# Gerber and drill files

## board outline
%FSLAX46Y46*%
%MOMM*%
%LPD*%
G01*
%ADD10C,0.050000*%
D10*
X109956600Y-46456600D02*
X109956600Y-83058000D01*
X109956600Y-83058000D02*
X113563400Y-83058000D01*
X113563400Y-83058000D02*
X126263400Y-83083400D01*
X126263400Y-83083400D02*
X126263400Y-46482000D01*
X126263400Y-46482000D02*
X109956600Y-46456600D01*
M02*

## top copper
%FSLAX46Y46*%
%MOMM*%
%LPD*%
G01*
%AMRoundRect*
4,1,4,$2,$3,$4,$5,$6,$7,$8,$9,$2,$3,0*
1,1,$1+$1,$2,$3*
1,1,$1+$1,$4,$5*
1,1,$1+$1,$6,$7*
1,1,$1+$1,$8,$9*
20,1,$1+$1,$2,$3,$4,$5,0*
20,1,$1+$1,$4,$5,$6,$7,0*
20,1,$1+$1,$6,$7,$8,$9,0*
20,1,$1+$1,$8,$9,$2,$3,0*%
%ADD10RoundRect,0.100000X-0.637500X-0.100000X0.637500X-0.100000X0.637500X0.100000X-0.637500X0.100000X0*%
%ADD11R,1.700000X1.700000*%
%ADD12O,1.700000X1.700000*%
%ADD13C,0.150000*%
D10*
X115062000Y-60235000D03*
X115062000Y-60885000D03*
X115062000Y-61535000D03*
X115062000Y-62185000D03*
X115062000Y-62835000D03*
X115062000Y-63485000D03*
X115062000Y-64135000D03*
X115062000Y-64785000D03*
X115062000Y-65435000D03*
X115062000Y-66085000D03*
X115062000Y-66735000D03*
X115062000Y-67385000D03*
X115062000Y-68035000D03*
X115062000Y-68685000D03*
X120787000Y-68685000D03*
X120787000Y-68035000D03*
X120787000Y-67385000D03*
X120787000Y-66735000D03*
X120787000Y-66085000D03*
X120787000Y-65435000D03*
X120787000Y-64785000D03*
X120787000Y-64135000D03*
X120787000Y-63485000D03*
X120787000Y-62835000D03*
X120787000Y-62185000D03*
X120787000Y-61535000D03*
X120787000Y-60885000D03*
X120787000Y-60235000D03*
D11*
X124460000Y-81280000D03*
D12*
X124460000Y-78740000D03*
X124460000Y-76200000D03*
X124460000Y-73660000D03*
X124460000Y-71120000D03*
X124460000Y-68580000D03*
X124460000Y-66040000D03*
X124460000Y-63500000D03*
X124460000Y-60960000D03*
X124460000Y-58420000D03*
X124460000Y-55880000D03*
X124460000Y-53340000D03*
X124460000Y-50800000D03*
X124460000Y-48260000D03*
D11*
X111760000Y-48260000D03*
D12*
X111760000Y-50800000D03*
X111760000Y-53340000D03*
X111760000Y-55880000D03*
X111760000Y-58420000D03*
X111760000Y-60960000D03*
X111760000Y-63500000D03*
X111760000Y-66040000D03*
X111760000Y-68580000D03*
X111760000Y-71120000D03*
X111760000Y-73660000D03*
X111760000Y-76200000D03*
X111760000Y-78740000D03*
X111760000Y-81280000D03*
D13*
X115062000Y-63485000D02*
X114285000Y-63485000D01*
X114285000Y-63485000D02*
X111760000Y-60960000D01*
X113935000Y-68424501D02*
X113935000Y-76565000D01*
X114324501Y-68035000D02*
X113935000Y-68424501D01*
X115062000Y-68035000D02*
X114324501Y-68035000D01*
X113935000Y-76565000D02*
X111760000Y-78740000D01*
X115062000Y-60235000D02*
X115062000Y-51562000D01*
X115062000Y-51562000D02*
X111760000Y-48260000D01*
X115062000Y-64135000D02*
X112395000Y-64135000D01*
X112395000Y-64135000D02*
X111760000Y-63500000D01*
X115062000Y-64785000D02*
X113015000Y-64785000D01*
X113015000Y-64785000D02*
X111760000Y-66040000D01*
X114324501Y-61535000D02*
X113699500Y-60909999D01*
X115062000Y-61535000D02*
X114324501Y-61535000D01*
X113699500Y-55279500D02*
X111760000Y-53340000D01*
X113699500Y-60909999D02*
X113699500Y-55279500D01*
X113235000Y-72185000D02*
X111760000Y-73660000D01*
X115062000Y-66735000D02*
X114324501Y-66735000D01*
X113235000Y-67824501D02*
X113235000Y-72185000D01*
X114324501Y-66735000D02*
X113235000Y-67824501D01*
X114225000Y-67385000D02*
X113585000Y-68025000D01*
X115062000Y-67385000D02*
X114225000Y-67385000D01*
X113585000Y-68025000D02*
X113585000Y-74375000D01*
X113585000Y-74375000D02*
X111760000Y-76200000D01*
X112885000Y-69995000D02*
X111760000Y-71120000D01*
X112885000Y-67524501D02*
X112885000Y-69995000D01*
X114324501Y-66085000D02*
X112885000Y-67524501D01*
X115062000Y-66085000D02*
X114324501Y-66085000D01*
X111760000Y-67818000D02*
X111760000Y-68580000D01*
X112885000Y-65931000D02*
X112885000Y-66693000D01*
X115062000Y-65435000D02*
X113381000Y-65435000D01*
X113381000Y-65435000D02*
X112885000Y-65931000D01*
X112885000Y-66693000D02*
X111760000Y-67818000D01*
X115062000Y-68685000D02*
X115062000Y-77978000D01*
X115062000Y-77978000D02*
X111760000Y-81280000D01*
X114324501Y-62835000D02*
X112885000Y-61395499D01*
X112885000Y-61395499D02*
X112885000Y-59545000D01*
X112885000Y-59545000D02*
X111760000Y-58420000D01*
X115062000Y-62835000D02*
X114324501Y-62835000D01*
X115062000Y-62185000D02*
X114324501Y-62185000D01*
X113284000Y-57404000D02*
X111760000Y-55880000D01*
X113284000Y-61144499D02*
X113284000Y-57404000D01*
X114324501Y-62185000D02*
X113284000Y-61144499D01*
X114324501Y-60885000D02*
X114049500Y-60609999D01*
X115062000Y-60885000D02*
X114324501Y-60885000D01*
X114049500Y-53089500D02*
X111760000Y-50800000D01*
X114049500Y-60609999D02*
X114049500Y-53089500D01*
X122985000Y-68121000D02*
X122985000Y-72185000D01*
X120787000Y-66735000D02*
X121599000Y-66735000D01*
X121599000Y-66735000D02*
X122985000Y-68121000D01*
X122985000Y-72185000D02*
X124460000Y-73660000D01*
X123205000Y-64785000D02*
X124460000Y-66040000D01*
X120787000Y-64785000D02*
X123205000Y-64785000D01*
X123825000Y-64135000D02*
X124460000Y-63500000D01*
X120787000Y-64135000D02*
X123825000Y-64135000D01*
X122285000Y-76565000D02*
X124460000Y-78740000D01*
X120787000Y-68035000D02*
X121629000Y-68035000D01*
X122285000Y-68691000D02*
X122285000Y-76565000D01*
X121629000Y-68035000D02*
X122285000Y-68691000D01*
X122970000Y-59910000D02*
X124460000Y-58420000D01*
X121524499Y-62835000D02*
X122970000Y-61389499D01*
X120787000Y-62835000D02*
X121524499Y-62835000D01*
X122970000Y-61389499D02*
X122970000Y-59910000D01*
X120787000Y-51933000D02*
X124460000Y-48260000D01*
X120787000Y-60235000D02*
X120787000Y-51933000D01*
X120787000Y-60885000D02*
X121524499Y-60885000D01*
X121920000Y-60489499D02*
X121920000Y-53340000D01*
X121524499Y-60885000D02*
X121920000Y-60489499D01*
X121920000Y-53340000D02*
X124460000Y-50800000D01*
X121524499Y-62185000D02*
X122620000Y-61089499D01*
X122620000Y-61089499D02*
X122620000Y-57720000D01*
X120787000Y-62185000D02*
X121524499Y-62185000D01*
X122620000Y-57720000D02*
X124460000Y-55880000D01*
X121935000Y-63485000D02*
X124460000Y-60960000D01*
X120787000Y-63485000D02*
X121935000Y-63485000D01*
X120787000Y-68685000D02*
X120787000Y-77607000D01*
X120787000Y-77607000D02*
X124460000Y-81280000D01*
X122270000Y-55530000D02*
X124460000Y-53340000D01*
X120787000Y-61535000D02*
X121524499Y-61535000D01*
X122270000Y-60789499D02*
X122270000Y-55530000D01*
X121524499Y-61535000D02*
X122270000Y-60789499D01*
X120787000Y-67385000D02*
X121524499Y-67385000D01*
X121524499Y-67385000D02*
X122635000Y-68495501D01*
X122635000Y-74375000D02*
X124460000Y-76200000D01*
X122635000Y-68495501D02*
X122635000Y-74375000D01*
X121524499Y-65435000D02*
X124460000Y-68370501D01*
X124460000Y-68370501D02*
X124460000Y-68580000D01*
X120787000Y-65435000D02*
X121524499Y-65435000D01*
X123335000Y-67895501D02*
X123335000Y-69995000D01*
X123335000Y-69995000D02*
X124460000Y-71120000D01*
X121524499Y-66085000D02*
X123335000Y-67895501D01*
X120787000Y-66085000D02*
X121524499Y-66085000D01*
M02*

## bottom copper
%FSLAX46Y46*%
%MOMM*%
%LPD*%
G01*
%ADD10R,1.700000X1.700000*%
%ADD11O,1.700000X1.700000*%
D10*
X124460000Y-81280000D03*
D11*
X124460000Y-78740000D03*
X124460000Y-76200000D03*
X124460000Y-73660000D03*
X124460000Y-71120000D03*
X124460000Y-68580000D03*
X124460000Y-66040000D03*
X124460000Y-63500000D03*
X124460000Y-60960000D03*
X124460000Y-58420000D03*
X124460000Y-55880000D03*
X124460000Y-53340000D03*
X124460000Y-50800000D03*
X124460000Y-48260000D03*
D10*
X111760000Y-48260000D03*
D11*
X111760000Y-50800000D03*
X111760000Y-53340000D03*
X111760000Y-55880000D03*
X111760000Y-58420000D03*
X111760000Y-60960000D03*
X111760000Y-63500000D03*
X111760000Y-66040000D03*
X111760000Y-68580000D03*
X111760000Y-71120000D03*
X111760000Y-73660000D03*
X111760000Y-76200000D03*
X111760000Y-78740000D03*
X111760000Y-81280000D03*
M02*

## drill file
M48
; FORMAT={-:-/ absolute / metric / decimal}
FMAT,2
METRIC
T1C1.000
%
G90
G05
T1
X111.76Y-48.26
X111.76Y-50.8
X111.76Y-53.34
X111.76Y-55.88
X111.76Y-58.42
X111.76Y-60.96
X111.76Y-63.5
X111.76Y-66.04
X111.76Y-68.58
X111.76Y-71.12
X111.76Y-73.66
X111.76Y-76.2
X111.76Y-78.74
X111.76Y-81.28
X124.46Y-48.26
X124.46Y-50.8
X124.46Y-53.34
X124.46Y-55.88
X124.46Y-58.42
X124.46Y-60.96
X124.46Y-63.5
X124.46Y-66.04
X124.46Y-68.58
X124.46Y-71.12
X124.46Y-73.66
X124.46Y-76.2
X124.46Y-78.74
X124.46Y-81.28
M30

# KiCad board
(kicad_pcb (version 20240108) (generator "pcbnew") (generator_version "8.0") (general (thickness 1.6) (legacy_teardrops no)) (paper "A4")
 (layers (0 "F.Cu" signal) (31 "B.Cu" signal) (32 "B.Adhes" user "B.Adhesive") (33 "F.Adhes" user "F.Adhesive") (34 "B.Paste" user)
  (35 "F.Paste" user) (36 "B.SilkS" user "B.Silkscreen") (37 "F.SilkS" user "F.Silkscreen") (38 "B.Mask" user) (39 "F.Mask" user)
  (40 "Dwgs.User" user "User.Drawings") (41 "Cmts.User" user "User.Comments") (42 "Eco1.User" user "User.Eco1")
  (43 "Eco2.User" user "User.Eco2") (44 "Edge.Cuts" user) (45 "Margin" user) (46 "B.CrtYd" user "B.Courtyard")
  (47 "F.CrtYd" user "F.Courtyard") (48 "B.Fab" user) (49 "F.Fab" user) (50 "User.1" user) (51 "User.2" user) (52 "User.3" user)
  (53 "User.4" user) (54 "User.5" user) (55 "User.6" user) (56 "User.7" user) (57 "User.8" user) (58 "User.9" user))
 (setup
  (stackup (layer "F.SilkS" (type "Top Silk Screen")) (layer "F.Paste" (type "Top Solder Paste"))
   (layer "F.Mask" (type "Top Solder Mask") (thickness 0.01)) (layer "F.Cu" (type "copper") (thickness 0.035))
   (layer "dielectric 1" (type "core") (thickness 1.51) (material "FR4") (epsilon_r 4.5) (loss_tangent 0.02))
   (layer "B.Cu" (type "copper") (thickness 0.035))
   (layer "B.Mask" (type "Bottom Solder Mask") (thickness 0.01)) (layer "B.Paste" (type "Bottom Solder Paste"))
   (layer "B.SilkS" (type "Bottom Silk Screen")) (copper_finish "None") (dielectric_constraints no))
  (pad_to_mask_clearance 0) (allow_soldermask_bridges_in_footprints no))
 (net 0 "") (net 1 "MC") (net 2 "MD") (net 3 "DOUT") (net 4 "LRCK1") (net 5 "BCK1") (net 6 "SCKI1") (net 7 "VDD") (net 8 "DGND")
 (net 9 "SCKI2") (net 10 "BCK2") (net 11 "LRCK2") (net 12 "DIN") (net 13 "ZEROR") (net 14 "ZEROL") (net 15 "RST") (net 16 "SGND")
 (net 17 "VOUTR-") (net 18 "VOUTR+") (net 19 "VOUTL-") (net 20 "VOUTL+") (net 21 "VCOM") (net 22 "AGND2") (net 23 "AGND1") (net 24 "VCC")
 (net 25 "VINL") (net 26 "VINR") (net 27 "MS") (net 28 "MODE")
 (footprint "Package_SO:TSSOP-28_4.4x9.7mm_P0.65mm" (layer "F.Cu") (at 117.9245 64.46)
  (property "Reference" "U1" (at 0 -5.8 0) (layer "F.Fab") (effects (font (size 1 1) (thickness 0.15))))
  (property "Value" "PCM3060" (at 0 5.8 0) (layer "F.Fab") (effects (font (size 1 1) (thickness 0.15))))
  (pad "1" smd roundrect (at -2.8625 -4.225) (size 1.475 0.4) (layers "F.Cu" "F.Paste" "F.Mask") (roundrect_rratio 0.25) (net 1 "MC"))
  (pad "2" smd roundrect (at -2.8625 -3.575) (size 1.475 0.4) (layers "F.Cu" "F.Paste" "F.Mask") (roundrect_rratio 0.25) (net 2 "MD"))
  (pad "3" smd roundrect (at -2.8625 -2.925) (size 1.475 0.4) (layers "F.Cu" "F.Paste" "F.Mask") (roundrect_rratio 0.25) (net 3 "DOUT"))
  (pad "4" smd roundrect (at -2.8625 -2.275) (size 1.475 0.4) (layers "F.Cu" "F.Paste" "F.Mask") (roundrect_rratio 0.25) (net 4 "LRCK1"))
  (pad "5" smd roundrect (at -2.8625 -1.625) (size 1.475 0.4) (layers "F.Cu" "F.Paste" "F.Mask") (roundrect_rratio 0.25) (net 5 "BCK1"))
  (pad "6" smd roundrect (at -2.8625 -0.975) (size 1.475 0.4) (layers "F.Cu" "F.Paste" "F.Mask") (roundrect_rratio 0.25) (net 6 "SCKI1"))
  (pad "7" smd roundrect (at -2.8625 -0.325) (size 1.475 0.4) (layers "F.Cu" "F.Paste" "F.Mask") (roundrect_rratio 0.25) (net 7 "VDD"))
  (pad "8" smd roundrect (at -2.8625 0.325) (size 1.475 0.4) (layers "F.Cu" "F.Paste" "F.Mask") (roundrect_rratio 0.25) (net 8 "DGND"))
  (pad "9" smd roundrect (at -2.8625 0.975) (size 1.475 0.4) (layers "F.Cu" "F.Paste" "F.Mask") (roundrect_rratio 0.25) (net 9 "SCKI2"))
  (pad "10" smd roundrect (at -2.8625 1.625) (size 1.475 0.4) (layers "F.Cu" "F.Paste" "F.Mask") (roundrect_rratio 0.25) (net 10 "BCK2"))
  (pad "11" smd roundrect (at -2.8625 2.275) (size 1.475 0.4) (layers "F.Cu" "F.Paste" "F.Mask") (roundrect_rratio 0.25) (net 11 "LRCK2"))
  (pad "12" smd roundrect (at -2.8625 2.925) (size 1.475 0.4) (layers "F.Cu" "F.Paste" "F.Mask") (roundrect_rratio 0.25) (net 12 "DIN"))
  (pad "13" smd roundrect (at -2.8625 3.575) (size 1.475 0.4) (layers "F.Cu" "F.Paste" "F.Mask") (roundrect_rratio 0.25) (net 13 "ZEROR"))
  (pad "14" smd roundrect (at -2.8625 4.225) (size 1.475 0.4) (layers "F.Cu" "F.Paste" "F.Mask") (roundrect_rratio 0.25) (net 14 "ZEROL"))
  (pad "15" smd roundrect (at 2.8625 4.225) (size 1.475 0.4) (layers "F.Cu" "F.Paste" "F.Mask") (roundrect_rratio 0.25) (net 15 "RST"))
  (pad "16" smd roundrect (at 2.8625 3.575) (size 1.475 0.4) (layers "F.Cu" "F.Paste" "F.Mask") (roundrect_rratio 0.25) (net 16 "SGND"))
  (pad "17" smd roundrect (at 2.8625 2.925) (size 1.475 0.4) (layers "F.Cu" "F.Paste" "F.Mask") (roundrect_rratio 0.25) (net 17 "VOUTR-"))
  (pad "18" smd roundrect (at 2.8625 2.275) (size 1.475 0.4) (layers "F.Cu" "F.Paste" "F.Mask") (roundrect_rratio 0.25) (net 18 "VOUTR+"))
  (pad "19" smd roundrect (at 2.8625 1.625) (size 1.475 0.4) (layers "F.Cu" "F.Paste" "F.Mask") (roundrect_rratio 0.25) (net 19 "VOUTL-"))
  (pad "20" smd roundrect (at 2.8625 0.975) (size 1.475 0.4) (layers "F.Cu" "F.Paste" "F.Mask") (roundrect_rratio 0.25) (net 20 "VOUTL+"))
  (pad "21" smd roundrect (at 2.8625 0.325) (size 1.475 0.4) (layers "F.Cu" "F.Paste" "F.Mask") (roundrect_rratio 0.25) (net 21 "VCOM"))
  (pad "22" smd roundrect (at 2.8625 -0.325) (size 1.475 0.4) (layers "F.Cu" "F.Paste" "F.Mask") (roundrect_rratio 0.25) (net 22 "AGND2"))
  (pad "23" smd roundrect (at 2.8625 -0.975) (size 1.475 0.4) (layers "F.Cu" "F.Paste" "F.Mask") (roundrect_rratio 0.25) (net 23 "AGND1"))
  (pad "24" smd roundrect (at 2.8625 -1.625) (size 1.475 0.4) (layers "F.Cu" "F.Paste" "F.Mask") (roundrect_rratio 0.25) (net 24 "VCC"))
  (pad "25" smd roundrect (at 2.8625 -2.275) (size 1.475 0.4) (layers "F.Cu" "F.Paste" "F.Mask") (roundrect_rratio 0.25) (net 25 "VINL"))
  (pad "26" smd roundrect (at 2.8625 -2.925) (size 1.475 0.4) (layers "F.Cu" "F.Paste" "F.Mask") (roundrect_rratio 0.25) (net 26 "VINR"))
  (pad "27" smd roundrect (at 2.8625 -3.575) (size 1.475 0.4) (layers "F.Cu" "F.Paste" "F.Mask") (roundrect_rratio 0.25) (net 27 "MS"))
  (pad "28" smd roundrect (at 2.8625 -4.225) (size 1.475 0.4) (layers "F.Cu" "F.Paste" "F.Mask") (roundrect_rratio 0.25) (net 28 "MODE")))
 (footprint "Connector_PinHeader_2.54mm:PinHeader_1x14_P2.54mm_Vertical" (layer "B.Cu") (at 124.46 81.28)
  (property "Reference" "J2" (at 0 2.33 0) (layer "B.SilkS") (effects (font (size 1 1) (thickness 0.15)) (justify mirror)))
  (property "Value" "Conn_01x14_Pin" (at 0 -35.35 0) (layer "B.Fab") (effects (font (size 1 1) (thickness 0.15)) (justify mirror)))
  (pad "1" thru_hole rect (at 0 0) (size 1.7 1.7) (drill 1) (layers "*.Cu" "*.Mask") (remove_unused_layers no) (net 15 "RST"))
  (pad "2" thru_hole oval (at 0 -2.54) (size 1.7 1.7) (drill 1) (layers "*.Cu" "*.Mask") (remove_unused_layers no) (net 16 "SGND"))
  (pad "3" thru_hole oval (at 0 -5.08) (size 1.7 1.7) (drill 1) (layers "*.Cu" "*.Mask") (remove_unused_layers no) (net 17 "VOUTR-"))
  (pad "4" thru_hole oval (at 0 -7.62) (size 1.7 1.7) (drill 1) (layers "*.Cu" "*.Mask") (remove_unused_layers no) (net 18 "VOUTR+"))
  (pad "5" thru_hole oval (at 0 -10.16) (size 1.7 1.7) (drill 1) (layers "*.Cu" "*.Mask") (remove_unused_layers no) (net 19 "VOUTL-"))
  (pad "6" thru_hole oval (at 0 -12.7) (size 1.7 1.7) (drill 1) (layers "*.Cu" "*.Mask") (remove_unused_layers no) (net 20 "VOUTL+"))
  (pad "7" thru_hole oval (at 0 -15.24) (size 1.7 1.7) (drill 1) (layers "*.Cu" "*.Mask") (remove_unused_layers no) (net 21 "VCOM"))
  (pad "8" thru_hole oval (at 0 -17.78) (size 1.7 1.7) (drill 1) (layers "*.Cu" "*.Mask") (remove_unused_layers no) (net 22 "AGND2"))
  (pad "9" thru_hole oval (at 0 -20.32) (size 1.7 1.7) (drill 1) (layers "*.Cu" "*.Mask") (remove_unused_layers no) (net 23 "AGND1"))
  (pad "10" thru_hole oval (at 0 -22.86) (size 1.7 1.7) (drill 1) (layers "*.Cu" "*.Mask") (remove_unused_layers no) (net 24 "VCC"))
  (pad "11" thru_hole oval (at 0 -25.4) (size 1.7 1.7) (drill 1) (layers "*.Cu" "*.Mask") (remove_unused_layers no) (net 25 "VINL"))
  (pad "12" thru_hole oval (at 0 -27.94) (size 1.7 1.7) (drill 1) (layers "*.Cu" "*.Mask") (remove_unused_layers no) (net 26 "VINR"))
  (pad "13" thru_hole oval (at 0 -30.48) (size 1.7 1.7) (drill 1) (layers "*.Cu" "*.Mask") (remove_unused_layers no) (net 27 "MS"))
  (pad "14" thru_hole oval (at 0 -33.02) (size 1.7 1.7) (drill 1) (layers "*.Cu" "*.Mask") (remove_unused_layers no) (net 28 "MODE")))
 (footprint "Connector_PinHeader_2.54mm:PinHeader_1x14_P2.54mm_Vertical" (layer "B.Cu") (at 111.76 48.26 180)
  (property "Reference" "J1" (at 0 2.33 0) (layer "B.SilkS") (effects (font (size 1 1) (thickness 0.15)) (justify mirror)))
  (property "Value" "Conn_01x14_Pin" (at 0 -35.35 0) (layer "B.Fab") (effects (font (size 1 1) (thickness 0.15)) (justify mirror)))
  (pad "1" thru_hole rect (at 0 0 180) (size 1.7 1.7) (drill 1) (layers "*.Cu" "*.Mask") (remove_unused_layers no) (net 1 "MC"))
  (pad "2" thru_hole oval (at 0 -2.54 180) (size 1.7 1.7) (drill 1) (layers "*.Cu" "*.Mask") (remove_unused_layers no) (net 2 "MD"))
  (pad "3" thru_hole oval (at 0 -5.08 180) (size 1.7 1.7) (drill 1) (layers "*.Cu" "*.Mask") (remove_unused_layers no) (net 3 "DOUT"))
  (pad "4" thru_hole oval (at 0 -7.62 180) (size 1.7 1.7) (drill 1) (layers "*.Cu" "*.Mask") (remove_unused_layers no) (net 4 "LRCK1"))
  (pad "5" thru_hole oval (at 0 -10.16 180) (size 1.7 1.7) (drill 1) (layers "*.Cu" "*.Mask") (remove_unused_layers no) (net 5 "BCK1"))
  (pad "6" thru_hole oval (at 0 -12.7 180) (size 1.7 1.7) (drill 1) (layers "*.Cu" "*.Mask") (remove_unused_layers no) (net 6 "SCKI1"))
  (pad "7" thru_hole oval (at 0 -15.24 180) (size 1.7 1.7) (drill 1) (layers "*.Cu" "*.Mask") (remove_unused_layers no) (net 7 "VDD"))
  (pad "8" thru_hole oval (at 0 -17.78 180) (size 1.7 1.7) (drill 1) (layers "*.Cu" "*.Mask") (remove_unused_layers no) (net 8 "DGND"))
  (pad "9" thru_hole oval (at 0 -20.32 180) (size 1.7 1.7) (drill 1) (layers "*.Cu" "*.Mask") (remove_unused_layers no) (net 9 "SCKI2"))
  (pad "10" thru_hole oval (at 0 -22.86 180) (size 1.7 1.7) (drill 1) (layers "*.Cu" "*.Mask") (remove_unused_layers no) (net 10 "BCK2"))
  (pad "11" thru_hole oval (at 0 -25.4 180) (size 1.7 1.7) (drill 1) (layers "*.Cu" "*.Mask") (remove_unused_layers no) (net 11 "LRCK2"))
  (pad "12" thru_hole oval (at 0 -27.94 180) (size 1.7 1.7) (drill 1) (layers "*.Cu" "*.Mask") (remove_unused_layers no) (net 12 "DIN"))
  (pad "13" thru_hole oval (at 0 -30.48 180) (size 1.7 1.7) (drill 1) (layers "*.Cu" "*.Mask") (remove_unused_layers no) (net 13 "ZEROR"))
  (pad "14" thru_hole oval (at 0 -33.02 180) (size 1.7 1.7) (drill 1) (layers "*.Cu" "*.Mask") (remove_unused_layers no) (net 14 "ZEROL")))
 (gr_line (start 109.9566 46.4566) (end 109.9566 83.058) (stroke (width 0.05) (type default)) (layer "Edge.Cuts"))
 (gr_line (start 109.9566 83.058) (end 113.5634 83.058) (stroke (width 0.05) (type default)) (layer "Edge.Cuts"))
 (gr_line (start 113.5634 83.058) (end 126.2634 83.0834) (stroke (width 0.05) (type default)) (layer "Edge.Cuts"))
 (gr_line (start 126.2634 83.0834) (end 126.2634 46.482) (stroke (width 0.05) (type default)) (layer "Edge.Cuts"))
 (gr_line (start 126.2634 46.482) (end 109.9566 46.4566) (stroke (width 0.05) (type default)) (layer "Edge.Cuts"))
 (segment (start 115.062 63.485) (end 114.285 63.485) (width 0.15) (layer "F.Cu") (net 6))
 (segment (start 114.285 63.485) (end 111.76 60.96) (width 0.15) (layer "F.Cu") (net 6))
 (segment (start 113.935 68.424501) (end 113.935 76.565) (width 0.15) (layer "F.Cu") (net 13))
 (segment (start 114.324501 68.035) (end 113.935 68.424501) (width 0.15) (layer "F.Cu") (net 13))
 (segment (start 115.062 68.035) (end 114.324501 68.035) (width 0.15) (layer "F.Cu") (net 13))
 (segment (start 113.935 76.565) (end 111.76 78.74) (width 0.15) (layer "F.Cu") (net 13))
 (segment (start 115.062 60.235) (end 115.062 51.562) (width 0.15) (layer "F.Cu") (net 1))
 (segment (start 115.062 51.562) (end 111.76 48.26) (width 0.15) (layer "F.Cu") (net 1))
 (segment (start 115.062 64.135) (end 112.395 64.135) (width 0.15) (layer "F.Cu") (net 7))
 (segment (start 112.395 64.135) (end 111.76 63.5) (width 0.15) (layer "F.Cu") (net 7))
 (segment (start 115.062 64.785) (end 113.015 64.785) (width 0.15) (layer "F.Cu") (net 8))
 (segment (start 113.015 64.785) (end 111.76 66.04) (width 0.15) (layer "F.Cu") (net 8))
 (segment (start 114.324501 61.535) (end 113.6995 60.909999) (width 0.15) (layer "F.Cu") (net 3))
 (segment (start 115.062 61.535) (end 114.324501 61.535) (width 0.15) (layer "F.Cu") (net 3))
 (segment (start 113.6995 55.2795) (end 111.76 53.34) (width 0.15) (layer "F.Cu") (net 3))
 (segment (start 113.6995 60.909999) (end 113.6995 55.2795) (width 0.15) (layer "F.Cu") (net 3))
 (segment (start 113.235 72.185) (end 111.76 73.66) (width 0.15) (layer "F.Cu") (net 11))
 (segment (start 115.062 66.735) (end 114.324501 66.735) (width 0.15) (layer "F.Cu") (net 11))
 (segment (start 113.235 67.824501) (end 113.235 72.185) (width 0.15) (layer "F.Cu") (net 11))
 (segment (start 114.324501 66.735) (end 113.235 67.824501) (width 0.15) (layer "F.Cu") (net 11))
 (segment (start 114.225 67.385) (end 113.585 68.025) (width 0.15) (layer "F.Cu") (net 12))
 (segment (start 115.062 67.385) (end 114.225 67.385) (width 0.15) (layer "F.Cu") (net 12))
 (segment (start 113.585 68.025) (end 113.585 74.375) (width 0.15) (layer "F.Cu") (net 12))
 (segment (start 113.585 74.375) (end 111.76 76.2) (width 0.15) (layer "F.Cu") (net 12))
 (segment (start 112.885 69.995) (end 111.76 71.12) (width 0.15) (layer "F.Cu") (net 10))
 (segment (start 112.885 67.524501) (end 112.885 69.995) (width 0.15) (layer "F.Cu") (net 10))
 (segment (start 114.324501 66.085) (end 112.885 67.524501) (width 0.15) (layer "F.Cu") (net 10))
 (segment (start 115.062 66.085) (end 114.324501 66.085) (width 0.15) (layer "F.Cu") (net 10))
 (segment (start 111.76 67.818) (end 111.76 68.58) (width 0.15) (layer "F.Cu") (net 9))
 (segment (start 112.885 65.931) (end 112.885 66.693) (width 0.15) (layer "F.Cu") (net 9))
 (segment (start 115.062 65.435) (end 113.381 65.435) (width 0.15) (layer "F.Cu") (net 9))
 (segment (start 113.381 65.435) (end 112.885 65.931) (width 0.15) (layer "F.Cu") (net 9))
 (segment (start 112.885 66.693) (end 111.76 67.818) (width 0.15) (layer "F.Cu") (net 9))
 (segment (start 115.062 68.685) (end 115.062 77.978) (width 0.15) (layer "F.Cu") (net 14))
 (segment (start 115.062 77.978) (end 111.76 81.28) (width 0.15) (layer "F.Cu") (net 14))
 (segment (start 114.324501 62.835) (end 112.885 61.395499) (width 0.15) (layer "F.Cu") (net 5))
 (segment (start 112.885 61.395499) (end 112.885 59.545) (width 0.15) (layer "F.Cu") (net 5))
 (segment (start 112.885 59.545) (end 111.76 58.42) (width 0.15) (layer "F.Cu") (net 5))
 (segment (start 115.062 62.835) (end 114.324501 62.835) (width 0.15) (layer "F.Cu") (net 5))
 (segment (start 115.062 62.185) (end 114.324501 62.185) (width 0.15) (layer "F.Cu") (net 4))
 (segment (start 113.284 57.404) (end 111.76 55.88) (width 0.15) (layer "F.Cu") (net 4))
 (segment (start 113.284 61.144499) (end 113.284 57.404) (width 0.15) (layer "F.Cu") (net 4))
 (segment (start 114.324501 62.185) (end 113.284 61.144499) (width 0.15) (layer "F.Cu") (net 4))
 (segment (start 114.324501 60.885) (end 114.0495 60.609999) (width 0.15) (layer "F.Cu") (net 2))
 (segment (start 115.062 60.885) (end 114.324501 60.885) (width 0.15) (layer "F.Cu") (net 2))
 (segment (start 114.0495 53.0895) (end 111.76 50.8) (width 0.15) (layer "F.Cu") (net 2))
 (segment (start 114.0495 60.609999) (end 114.0495 53.0895) (width 0.15) (layer "F.Cu") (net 2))
 (segment (start 122.985 68.121) (end 122.985 72.185) (width 0.15) (layer "F.Cu") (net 18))
 (segment (start 120.787 66.735) (end 121.599 66.735) (width 0.15) (layer "F.Cu") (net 18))
 (segment (start 121.599 66.735) (end 122.985 68.121) (width 0.15) (layer "F.Cu") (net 18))
 (segment (start 122.985 72.185) (end 124.46 73.66) (width 0.15) (layer "F.Cu") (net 18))
 (segment (start 123.205 64.785) (end 124.46 66.04) (width 0.15) (layer "F.Cu") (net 21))
 (segment (start 120.787 64.785) (end 123.205 64.785) (width 0.15) (layer "F.Cu") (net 21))
 (segment (start 123.825 64.135) (end 124.46 63.5) (width 0.15) (layer "F.Cu") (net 22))
 (segment (start 120.787 64.135) (end 123.825 64.135) (width 0.15) (layer "F.Cu") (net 22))
 (segment (start 122.285 76.565) (end 124.46 78.74) (width 0.15) (layer "F.Cu") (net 16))
 (segment (start 120.787 68.035) (end 121.629 68.035) (width 0.15) (layer "F.Cu") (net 16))
 (segment (start 122.285 68.691) (end 122.285 76.565) (width 0.15) (layer "F.Cu") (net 16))
 (segment (start 121.629 68.035) (end 122.285 68.691) (width 0.15) (layer "F.Cu") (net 16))
 (segment (start 122.97 59.91) (end 124.46 58.42) (width 0.15) (layer "F.Cu") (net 24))
 (segment (start 121.524499 62.835) (end 122.97 61.389499) (width 0.15) (layer "F.Cu") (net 24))
 (segment (start 120.787 62.835) (end 121.524499 62.835) (width 0.15) (layer "F.Cu") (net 24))
 (segment (start 122.97 61.389499) (end 122.97 59.91) (width 0.15) (layer "F.Cu") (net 24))
 (segment (start 120.787 51.933) (end 124.46 48.26) (width 0.15) (layer "F.Cu") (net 28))
 (segment (start 120.787 60.235) (end 120.787 51.933) (width 0.15) (layer "F.Cu") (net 28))
 (segment (start 120.787 60.885) (end 121.524499 60.885) (width 0.15) (layer "F.Cu") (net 27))
 (segment (start 121.92 60.489499) (end 121.92 53.34) (width 0.15) (layer "F.Cu") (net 27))
 (segment (start 121.524499 60.885) (end 121.92 60.489499) (width 0.15) (layer "F.Cu") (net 27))
 (segment (start 121.92 53.34) (end 124.46 50.8) (width 0.15) (layer "F.Cu") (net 27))
 (segment (start 121.524499 62.185) (end 122.62 61.089499) (width 0.15) (layer "F.Cu") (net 25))
 (segment (start 122.62 61.089499) (end 122.62 57.72) (width 0.15) (layer "F.Cu") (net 25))
 (segment (start 120.787 62.185) (end 121.524499 62.185) (width 0.15) (layer "F.Cu") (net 25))
 (segment (start 122.62 57.72) (end 124.46 55.88) (width 0.15) (layer "F.Cu") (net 25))
 (segment (start 121.935 63.485) (end 124.46 60.96) (width 0.15) (layer "F.Cu") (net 23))
 (segment (start 120.787 63.485) (end 121.935 63.485) (width 0.15) (layer "F.Cu") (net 23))
 (segment (start 120.787 68.685) (end 120.787 77.607) (width 0.15) (layer "F.Cu") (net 15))
 (segment (start 120.787 77.607) (end 124.46 81.28) (width 0.15) (layer "F.Cu") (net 15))
 (segment (start 122.27 55.53) (end 124.46 53.34) (width 0.15) (layer "F.Cu") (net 26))
 (segment (start 120.787 61.535) (end 121.524499 61.535) (width 0.15) (layer "F.Cu") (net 26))
 (segment (start 122.27 60.789499) (end 122.27 55.53) (width 0.15) (layer "F.Cu") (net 26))
 (segment (start 121.524499 61.535) (end 122.27 60.789499) (width 0.15) (layer "F.Cu") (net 26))
 (segment (start 120.787 67.385) (end 121.524499 67.385) (width 0.15) (layer "F.Cu") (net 17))
 (segment (start 121.524499 67.385) (end 122.635 68.495501) (width 0.15) (layer "F.Cu") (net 17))
 (segment (start 122.635 74.375) (end 124.46 76.2) (width 0.15) (layer "F.Cu") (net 17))
 (segment (start 122.635 68.495501) (end 122.635 74.375) (width 0.15) (layer "F.Cu") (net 17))
 (segment (start 121.524499 65.435) (end 124.46 68.370501) (width 0.15) (layer "F.Cu") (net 20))
 (segment (start 124.46 68.370501) (end 124.46 68.58) (width 0.15) (layer "F.Cu") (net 20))
 (segment (start 120.787 65.435) (end 121.524499 65.435) (width 0.15) (layer "F.Cu") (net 20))
 (segment (start 123.335 67.895501) (end 123.335 69.995) (width 0.15) (layer "F.Cu") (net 19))
 (segment (start 123.335 69.995) (end 124.46 71.12) (width 0.15) (layer "F.Cu") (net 19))
 (segment (start 121.524499 66.085) (end 123.335 67.895501) (width 0.15) (layer "F.Cu") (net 19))
 (segment (start 120.787 66.085) (end 121.524499 66.085) (width 0.15) (layer "F.Cu") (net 19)))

